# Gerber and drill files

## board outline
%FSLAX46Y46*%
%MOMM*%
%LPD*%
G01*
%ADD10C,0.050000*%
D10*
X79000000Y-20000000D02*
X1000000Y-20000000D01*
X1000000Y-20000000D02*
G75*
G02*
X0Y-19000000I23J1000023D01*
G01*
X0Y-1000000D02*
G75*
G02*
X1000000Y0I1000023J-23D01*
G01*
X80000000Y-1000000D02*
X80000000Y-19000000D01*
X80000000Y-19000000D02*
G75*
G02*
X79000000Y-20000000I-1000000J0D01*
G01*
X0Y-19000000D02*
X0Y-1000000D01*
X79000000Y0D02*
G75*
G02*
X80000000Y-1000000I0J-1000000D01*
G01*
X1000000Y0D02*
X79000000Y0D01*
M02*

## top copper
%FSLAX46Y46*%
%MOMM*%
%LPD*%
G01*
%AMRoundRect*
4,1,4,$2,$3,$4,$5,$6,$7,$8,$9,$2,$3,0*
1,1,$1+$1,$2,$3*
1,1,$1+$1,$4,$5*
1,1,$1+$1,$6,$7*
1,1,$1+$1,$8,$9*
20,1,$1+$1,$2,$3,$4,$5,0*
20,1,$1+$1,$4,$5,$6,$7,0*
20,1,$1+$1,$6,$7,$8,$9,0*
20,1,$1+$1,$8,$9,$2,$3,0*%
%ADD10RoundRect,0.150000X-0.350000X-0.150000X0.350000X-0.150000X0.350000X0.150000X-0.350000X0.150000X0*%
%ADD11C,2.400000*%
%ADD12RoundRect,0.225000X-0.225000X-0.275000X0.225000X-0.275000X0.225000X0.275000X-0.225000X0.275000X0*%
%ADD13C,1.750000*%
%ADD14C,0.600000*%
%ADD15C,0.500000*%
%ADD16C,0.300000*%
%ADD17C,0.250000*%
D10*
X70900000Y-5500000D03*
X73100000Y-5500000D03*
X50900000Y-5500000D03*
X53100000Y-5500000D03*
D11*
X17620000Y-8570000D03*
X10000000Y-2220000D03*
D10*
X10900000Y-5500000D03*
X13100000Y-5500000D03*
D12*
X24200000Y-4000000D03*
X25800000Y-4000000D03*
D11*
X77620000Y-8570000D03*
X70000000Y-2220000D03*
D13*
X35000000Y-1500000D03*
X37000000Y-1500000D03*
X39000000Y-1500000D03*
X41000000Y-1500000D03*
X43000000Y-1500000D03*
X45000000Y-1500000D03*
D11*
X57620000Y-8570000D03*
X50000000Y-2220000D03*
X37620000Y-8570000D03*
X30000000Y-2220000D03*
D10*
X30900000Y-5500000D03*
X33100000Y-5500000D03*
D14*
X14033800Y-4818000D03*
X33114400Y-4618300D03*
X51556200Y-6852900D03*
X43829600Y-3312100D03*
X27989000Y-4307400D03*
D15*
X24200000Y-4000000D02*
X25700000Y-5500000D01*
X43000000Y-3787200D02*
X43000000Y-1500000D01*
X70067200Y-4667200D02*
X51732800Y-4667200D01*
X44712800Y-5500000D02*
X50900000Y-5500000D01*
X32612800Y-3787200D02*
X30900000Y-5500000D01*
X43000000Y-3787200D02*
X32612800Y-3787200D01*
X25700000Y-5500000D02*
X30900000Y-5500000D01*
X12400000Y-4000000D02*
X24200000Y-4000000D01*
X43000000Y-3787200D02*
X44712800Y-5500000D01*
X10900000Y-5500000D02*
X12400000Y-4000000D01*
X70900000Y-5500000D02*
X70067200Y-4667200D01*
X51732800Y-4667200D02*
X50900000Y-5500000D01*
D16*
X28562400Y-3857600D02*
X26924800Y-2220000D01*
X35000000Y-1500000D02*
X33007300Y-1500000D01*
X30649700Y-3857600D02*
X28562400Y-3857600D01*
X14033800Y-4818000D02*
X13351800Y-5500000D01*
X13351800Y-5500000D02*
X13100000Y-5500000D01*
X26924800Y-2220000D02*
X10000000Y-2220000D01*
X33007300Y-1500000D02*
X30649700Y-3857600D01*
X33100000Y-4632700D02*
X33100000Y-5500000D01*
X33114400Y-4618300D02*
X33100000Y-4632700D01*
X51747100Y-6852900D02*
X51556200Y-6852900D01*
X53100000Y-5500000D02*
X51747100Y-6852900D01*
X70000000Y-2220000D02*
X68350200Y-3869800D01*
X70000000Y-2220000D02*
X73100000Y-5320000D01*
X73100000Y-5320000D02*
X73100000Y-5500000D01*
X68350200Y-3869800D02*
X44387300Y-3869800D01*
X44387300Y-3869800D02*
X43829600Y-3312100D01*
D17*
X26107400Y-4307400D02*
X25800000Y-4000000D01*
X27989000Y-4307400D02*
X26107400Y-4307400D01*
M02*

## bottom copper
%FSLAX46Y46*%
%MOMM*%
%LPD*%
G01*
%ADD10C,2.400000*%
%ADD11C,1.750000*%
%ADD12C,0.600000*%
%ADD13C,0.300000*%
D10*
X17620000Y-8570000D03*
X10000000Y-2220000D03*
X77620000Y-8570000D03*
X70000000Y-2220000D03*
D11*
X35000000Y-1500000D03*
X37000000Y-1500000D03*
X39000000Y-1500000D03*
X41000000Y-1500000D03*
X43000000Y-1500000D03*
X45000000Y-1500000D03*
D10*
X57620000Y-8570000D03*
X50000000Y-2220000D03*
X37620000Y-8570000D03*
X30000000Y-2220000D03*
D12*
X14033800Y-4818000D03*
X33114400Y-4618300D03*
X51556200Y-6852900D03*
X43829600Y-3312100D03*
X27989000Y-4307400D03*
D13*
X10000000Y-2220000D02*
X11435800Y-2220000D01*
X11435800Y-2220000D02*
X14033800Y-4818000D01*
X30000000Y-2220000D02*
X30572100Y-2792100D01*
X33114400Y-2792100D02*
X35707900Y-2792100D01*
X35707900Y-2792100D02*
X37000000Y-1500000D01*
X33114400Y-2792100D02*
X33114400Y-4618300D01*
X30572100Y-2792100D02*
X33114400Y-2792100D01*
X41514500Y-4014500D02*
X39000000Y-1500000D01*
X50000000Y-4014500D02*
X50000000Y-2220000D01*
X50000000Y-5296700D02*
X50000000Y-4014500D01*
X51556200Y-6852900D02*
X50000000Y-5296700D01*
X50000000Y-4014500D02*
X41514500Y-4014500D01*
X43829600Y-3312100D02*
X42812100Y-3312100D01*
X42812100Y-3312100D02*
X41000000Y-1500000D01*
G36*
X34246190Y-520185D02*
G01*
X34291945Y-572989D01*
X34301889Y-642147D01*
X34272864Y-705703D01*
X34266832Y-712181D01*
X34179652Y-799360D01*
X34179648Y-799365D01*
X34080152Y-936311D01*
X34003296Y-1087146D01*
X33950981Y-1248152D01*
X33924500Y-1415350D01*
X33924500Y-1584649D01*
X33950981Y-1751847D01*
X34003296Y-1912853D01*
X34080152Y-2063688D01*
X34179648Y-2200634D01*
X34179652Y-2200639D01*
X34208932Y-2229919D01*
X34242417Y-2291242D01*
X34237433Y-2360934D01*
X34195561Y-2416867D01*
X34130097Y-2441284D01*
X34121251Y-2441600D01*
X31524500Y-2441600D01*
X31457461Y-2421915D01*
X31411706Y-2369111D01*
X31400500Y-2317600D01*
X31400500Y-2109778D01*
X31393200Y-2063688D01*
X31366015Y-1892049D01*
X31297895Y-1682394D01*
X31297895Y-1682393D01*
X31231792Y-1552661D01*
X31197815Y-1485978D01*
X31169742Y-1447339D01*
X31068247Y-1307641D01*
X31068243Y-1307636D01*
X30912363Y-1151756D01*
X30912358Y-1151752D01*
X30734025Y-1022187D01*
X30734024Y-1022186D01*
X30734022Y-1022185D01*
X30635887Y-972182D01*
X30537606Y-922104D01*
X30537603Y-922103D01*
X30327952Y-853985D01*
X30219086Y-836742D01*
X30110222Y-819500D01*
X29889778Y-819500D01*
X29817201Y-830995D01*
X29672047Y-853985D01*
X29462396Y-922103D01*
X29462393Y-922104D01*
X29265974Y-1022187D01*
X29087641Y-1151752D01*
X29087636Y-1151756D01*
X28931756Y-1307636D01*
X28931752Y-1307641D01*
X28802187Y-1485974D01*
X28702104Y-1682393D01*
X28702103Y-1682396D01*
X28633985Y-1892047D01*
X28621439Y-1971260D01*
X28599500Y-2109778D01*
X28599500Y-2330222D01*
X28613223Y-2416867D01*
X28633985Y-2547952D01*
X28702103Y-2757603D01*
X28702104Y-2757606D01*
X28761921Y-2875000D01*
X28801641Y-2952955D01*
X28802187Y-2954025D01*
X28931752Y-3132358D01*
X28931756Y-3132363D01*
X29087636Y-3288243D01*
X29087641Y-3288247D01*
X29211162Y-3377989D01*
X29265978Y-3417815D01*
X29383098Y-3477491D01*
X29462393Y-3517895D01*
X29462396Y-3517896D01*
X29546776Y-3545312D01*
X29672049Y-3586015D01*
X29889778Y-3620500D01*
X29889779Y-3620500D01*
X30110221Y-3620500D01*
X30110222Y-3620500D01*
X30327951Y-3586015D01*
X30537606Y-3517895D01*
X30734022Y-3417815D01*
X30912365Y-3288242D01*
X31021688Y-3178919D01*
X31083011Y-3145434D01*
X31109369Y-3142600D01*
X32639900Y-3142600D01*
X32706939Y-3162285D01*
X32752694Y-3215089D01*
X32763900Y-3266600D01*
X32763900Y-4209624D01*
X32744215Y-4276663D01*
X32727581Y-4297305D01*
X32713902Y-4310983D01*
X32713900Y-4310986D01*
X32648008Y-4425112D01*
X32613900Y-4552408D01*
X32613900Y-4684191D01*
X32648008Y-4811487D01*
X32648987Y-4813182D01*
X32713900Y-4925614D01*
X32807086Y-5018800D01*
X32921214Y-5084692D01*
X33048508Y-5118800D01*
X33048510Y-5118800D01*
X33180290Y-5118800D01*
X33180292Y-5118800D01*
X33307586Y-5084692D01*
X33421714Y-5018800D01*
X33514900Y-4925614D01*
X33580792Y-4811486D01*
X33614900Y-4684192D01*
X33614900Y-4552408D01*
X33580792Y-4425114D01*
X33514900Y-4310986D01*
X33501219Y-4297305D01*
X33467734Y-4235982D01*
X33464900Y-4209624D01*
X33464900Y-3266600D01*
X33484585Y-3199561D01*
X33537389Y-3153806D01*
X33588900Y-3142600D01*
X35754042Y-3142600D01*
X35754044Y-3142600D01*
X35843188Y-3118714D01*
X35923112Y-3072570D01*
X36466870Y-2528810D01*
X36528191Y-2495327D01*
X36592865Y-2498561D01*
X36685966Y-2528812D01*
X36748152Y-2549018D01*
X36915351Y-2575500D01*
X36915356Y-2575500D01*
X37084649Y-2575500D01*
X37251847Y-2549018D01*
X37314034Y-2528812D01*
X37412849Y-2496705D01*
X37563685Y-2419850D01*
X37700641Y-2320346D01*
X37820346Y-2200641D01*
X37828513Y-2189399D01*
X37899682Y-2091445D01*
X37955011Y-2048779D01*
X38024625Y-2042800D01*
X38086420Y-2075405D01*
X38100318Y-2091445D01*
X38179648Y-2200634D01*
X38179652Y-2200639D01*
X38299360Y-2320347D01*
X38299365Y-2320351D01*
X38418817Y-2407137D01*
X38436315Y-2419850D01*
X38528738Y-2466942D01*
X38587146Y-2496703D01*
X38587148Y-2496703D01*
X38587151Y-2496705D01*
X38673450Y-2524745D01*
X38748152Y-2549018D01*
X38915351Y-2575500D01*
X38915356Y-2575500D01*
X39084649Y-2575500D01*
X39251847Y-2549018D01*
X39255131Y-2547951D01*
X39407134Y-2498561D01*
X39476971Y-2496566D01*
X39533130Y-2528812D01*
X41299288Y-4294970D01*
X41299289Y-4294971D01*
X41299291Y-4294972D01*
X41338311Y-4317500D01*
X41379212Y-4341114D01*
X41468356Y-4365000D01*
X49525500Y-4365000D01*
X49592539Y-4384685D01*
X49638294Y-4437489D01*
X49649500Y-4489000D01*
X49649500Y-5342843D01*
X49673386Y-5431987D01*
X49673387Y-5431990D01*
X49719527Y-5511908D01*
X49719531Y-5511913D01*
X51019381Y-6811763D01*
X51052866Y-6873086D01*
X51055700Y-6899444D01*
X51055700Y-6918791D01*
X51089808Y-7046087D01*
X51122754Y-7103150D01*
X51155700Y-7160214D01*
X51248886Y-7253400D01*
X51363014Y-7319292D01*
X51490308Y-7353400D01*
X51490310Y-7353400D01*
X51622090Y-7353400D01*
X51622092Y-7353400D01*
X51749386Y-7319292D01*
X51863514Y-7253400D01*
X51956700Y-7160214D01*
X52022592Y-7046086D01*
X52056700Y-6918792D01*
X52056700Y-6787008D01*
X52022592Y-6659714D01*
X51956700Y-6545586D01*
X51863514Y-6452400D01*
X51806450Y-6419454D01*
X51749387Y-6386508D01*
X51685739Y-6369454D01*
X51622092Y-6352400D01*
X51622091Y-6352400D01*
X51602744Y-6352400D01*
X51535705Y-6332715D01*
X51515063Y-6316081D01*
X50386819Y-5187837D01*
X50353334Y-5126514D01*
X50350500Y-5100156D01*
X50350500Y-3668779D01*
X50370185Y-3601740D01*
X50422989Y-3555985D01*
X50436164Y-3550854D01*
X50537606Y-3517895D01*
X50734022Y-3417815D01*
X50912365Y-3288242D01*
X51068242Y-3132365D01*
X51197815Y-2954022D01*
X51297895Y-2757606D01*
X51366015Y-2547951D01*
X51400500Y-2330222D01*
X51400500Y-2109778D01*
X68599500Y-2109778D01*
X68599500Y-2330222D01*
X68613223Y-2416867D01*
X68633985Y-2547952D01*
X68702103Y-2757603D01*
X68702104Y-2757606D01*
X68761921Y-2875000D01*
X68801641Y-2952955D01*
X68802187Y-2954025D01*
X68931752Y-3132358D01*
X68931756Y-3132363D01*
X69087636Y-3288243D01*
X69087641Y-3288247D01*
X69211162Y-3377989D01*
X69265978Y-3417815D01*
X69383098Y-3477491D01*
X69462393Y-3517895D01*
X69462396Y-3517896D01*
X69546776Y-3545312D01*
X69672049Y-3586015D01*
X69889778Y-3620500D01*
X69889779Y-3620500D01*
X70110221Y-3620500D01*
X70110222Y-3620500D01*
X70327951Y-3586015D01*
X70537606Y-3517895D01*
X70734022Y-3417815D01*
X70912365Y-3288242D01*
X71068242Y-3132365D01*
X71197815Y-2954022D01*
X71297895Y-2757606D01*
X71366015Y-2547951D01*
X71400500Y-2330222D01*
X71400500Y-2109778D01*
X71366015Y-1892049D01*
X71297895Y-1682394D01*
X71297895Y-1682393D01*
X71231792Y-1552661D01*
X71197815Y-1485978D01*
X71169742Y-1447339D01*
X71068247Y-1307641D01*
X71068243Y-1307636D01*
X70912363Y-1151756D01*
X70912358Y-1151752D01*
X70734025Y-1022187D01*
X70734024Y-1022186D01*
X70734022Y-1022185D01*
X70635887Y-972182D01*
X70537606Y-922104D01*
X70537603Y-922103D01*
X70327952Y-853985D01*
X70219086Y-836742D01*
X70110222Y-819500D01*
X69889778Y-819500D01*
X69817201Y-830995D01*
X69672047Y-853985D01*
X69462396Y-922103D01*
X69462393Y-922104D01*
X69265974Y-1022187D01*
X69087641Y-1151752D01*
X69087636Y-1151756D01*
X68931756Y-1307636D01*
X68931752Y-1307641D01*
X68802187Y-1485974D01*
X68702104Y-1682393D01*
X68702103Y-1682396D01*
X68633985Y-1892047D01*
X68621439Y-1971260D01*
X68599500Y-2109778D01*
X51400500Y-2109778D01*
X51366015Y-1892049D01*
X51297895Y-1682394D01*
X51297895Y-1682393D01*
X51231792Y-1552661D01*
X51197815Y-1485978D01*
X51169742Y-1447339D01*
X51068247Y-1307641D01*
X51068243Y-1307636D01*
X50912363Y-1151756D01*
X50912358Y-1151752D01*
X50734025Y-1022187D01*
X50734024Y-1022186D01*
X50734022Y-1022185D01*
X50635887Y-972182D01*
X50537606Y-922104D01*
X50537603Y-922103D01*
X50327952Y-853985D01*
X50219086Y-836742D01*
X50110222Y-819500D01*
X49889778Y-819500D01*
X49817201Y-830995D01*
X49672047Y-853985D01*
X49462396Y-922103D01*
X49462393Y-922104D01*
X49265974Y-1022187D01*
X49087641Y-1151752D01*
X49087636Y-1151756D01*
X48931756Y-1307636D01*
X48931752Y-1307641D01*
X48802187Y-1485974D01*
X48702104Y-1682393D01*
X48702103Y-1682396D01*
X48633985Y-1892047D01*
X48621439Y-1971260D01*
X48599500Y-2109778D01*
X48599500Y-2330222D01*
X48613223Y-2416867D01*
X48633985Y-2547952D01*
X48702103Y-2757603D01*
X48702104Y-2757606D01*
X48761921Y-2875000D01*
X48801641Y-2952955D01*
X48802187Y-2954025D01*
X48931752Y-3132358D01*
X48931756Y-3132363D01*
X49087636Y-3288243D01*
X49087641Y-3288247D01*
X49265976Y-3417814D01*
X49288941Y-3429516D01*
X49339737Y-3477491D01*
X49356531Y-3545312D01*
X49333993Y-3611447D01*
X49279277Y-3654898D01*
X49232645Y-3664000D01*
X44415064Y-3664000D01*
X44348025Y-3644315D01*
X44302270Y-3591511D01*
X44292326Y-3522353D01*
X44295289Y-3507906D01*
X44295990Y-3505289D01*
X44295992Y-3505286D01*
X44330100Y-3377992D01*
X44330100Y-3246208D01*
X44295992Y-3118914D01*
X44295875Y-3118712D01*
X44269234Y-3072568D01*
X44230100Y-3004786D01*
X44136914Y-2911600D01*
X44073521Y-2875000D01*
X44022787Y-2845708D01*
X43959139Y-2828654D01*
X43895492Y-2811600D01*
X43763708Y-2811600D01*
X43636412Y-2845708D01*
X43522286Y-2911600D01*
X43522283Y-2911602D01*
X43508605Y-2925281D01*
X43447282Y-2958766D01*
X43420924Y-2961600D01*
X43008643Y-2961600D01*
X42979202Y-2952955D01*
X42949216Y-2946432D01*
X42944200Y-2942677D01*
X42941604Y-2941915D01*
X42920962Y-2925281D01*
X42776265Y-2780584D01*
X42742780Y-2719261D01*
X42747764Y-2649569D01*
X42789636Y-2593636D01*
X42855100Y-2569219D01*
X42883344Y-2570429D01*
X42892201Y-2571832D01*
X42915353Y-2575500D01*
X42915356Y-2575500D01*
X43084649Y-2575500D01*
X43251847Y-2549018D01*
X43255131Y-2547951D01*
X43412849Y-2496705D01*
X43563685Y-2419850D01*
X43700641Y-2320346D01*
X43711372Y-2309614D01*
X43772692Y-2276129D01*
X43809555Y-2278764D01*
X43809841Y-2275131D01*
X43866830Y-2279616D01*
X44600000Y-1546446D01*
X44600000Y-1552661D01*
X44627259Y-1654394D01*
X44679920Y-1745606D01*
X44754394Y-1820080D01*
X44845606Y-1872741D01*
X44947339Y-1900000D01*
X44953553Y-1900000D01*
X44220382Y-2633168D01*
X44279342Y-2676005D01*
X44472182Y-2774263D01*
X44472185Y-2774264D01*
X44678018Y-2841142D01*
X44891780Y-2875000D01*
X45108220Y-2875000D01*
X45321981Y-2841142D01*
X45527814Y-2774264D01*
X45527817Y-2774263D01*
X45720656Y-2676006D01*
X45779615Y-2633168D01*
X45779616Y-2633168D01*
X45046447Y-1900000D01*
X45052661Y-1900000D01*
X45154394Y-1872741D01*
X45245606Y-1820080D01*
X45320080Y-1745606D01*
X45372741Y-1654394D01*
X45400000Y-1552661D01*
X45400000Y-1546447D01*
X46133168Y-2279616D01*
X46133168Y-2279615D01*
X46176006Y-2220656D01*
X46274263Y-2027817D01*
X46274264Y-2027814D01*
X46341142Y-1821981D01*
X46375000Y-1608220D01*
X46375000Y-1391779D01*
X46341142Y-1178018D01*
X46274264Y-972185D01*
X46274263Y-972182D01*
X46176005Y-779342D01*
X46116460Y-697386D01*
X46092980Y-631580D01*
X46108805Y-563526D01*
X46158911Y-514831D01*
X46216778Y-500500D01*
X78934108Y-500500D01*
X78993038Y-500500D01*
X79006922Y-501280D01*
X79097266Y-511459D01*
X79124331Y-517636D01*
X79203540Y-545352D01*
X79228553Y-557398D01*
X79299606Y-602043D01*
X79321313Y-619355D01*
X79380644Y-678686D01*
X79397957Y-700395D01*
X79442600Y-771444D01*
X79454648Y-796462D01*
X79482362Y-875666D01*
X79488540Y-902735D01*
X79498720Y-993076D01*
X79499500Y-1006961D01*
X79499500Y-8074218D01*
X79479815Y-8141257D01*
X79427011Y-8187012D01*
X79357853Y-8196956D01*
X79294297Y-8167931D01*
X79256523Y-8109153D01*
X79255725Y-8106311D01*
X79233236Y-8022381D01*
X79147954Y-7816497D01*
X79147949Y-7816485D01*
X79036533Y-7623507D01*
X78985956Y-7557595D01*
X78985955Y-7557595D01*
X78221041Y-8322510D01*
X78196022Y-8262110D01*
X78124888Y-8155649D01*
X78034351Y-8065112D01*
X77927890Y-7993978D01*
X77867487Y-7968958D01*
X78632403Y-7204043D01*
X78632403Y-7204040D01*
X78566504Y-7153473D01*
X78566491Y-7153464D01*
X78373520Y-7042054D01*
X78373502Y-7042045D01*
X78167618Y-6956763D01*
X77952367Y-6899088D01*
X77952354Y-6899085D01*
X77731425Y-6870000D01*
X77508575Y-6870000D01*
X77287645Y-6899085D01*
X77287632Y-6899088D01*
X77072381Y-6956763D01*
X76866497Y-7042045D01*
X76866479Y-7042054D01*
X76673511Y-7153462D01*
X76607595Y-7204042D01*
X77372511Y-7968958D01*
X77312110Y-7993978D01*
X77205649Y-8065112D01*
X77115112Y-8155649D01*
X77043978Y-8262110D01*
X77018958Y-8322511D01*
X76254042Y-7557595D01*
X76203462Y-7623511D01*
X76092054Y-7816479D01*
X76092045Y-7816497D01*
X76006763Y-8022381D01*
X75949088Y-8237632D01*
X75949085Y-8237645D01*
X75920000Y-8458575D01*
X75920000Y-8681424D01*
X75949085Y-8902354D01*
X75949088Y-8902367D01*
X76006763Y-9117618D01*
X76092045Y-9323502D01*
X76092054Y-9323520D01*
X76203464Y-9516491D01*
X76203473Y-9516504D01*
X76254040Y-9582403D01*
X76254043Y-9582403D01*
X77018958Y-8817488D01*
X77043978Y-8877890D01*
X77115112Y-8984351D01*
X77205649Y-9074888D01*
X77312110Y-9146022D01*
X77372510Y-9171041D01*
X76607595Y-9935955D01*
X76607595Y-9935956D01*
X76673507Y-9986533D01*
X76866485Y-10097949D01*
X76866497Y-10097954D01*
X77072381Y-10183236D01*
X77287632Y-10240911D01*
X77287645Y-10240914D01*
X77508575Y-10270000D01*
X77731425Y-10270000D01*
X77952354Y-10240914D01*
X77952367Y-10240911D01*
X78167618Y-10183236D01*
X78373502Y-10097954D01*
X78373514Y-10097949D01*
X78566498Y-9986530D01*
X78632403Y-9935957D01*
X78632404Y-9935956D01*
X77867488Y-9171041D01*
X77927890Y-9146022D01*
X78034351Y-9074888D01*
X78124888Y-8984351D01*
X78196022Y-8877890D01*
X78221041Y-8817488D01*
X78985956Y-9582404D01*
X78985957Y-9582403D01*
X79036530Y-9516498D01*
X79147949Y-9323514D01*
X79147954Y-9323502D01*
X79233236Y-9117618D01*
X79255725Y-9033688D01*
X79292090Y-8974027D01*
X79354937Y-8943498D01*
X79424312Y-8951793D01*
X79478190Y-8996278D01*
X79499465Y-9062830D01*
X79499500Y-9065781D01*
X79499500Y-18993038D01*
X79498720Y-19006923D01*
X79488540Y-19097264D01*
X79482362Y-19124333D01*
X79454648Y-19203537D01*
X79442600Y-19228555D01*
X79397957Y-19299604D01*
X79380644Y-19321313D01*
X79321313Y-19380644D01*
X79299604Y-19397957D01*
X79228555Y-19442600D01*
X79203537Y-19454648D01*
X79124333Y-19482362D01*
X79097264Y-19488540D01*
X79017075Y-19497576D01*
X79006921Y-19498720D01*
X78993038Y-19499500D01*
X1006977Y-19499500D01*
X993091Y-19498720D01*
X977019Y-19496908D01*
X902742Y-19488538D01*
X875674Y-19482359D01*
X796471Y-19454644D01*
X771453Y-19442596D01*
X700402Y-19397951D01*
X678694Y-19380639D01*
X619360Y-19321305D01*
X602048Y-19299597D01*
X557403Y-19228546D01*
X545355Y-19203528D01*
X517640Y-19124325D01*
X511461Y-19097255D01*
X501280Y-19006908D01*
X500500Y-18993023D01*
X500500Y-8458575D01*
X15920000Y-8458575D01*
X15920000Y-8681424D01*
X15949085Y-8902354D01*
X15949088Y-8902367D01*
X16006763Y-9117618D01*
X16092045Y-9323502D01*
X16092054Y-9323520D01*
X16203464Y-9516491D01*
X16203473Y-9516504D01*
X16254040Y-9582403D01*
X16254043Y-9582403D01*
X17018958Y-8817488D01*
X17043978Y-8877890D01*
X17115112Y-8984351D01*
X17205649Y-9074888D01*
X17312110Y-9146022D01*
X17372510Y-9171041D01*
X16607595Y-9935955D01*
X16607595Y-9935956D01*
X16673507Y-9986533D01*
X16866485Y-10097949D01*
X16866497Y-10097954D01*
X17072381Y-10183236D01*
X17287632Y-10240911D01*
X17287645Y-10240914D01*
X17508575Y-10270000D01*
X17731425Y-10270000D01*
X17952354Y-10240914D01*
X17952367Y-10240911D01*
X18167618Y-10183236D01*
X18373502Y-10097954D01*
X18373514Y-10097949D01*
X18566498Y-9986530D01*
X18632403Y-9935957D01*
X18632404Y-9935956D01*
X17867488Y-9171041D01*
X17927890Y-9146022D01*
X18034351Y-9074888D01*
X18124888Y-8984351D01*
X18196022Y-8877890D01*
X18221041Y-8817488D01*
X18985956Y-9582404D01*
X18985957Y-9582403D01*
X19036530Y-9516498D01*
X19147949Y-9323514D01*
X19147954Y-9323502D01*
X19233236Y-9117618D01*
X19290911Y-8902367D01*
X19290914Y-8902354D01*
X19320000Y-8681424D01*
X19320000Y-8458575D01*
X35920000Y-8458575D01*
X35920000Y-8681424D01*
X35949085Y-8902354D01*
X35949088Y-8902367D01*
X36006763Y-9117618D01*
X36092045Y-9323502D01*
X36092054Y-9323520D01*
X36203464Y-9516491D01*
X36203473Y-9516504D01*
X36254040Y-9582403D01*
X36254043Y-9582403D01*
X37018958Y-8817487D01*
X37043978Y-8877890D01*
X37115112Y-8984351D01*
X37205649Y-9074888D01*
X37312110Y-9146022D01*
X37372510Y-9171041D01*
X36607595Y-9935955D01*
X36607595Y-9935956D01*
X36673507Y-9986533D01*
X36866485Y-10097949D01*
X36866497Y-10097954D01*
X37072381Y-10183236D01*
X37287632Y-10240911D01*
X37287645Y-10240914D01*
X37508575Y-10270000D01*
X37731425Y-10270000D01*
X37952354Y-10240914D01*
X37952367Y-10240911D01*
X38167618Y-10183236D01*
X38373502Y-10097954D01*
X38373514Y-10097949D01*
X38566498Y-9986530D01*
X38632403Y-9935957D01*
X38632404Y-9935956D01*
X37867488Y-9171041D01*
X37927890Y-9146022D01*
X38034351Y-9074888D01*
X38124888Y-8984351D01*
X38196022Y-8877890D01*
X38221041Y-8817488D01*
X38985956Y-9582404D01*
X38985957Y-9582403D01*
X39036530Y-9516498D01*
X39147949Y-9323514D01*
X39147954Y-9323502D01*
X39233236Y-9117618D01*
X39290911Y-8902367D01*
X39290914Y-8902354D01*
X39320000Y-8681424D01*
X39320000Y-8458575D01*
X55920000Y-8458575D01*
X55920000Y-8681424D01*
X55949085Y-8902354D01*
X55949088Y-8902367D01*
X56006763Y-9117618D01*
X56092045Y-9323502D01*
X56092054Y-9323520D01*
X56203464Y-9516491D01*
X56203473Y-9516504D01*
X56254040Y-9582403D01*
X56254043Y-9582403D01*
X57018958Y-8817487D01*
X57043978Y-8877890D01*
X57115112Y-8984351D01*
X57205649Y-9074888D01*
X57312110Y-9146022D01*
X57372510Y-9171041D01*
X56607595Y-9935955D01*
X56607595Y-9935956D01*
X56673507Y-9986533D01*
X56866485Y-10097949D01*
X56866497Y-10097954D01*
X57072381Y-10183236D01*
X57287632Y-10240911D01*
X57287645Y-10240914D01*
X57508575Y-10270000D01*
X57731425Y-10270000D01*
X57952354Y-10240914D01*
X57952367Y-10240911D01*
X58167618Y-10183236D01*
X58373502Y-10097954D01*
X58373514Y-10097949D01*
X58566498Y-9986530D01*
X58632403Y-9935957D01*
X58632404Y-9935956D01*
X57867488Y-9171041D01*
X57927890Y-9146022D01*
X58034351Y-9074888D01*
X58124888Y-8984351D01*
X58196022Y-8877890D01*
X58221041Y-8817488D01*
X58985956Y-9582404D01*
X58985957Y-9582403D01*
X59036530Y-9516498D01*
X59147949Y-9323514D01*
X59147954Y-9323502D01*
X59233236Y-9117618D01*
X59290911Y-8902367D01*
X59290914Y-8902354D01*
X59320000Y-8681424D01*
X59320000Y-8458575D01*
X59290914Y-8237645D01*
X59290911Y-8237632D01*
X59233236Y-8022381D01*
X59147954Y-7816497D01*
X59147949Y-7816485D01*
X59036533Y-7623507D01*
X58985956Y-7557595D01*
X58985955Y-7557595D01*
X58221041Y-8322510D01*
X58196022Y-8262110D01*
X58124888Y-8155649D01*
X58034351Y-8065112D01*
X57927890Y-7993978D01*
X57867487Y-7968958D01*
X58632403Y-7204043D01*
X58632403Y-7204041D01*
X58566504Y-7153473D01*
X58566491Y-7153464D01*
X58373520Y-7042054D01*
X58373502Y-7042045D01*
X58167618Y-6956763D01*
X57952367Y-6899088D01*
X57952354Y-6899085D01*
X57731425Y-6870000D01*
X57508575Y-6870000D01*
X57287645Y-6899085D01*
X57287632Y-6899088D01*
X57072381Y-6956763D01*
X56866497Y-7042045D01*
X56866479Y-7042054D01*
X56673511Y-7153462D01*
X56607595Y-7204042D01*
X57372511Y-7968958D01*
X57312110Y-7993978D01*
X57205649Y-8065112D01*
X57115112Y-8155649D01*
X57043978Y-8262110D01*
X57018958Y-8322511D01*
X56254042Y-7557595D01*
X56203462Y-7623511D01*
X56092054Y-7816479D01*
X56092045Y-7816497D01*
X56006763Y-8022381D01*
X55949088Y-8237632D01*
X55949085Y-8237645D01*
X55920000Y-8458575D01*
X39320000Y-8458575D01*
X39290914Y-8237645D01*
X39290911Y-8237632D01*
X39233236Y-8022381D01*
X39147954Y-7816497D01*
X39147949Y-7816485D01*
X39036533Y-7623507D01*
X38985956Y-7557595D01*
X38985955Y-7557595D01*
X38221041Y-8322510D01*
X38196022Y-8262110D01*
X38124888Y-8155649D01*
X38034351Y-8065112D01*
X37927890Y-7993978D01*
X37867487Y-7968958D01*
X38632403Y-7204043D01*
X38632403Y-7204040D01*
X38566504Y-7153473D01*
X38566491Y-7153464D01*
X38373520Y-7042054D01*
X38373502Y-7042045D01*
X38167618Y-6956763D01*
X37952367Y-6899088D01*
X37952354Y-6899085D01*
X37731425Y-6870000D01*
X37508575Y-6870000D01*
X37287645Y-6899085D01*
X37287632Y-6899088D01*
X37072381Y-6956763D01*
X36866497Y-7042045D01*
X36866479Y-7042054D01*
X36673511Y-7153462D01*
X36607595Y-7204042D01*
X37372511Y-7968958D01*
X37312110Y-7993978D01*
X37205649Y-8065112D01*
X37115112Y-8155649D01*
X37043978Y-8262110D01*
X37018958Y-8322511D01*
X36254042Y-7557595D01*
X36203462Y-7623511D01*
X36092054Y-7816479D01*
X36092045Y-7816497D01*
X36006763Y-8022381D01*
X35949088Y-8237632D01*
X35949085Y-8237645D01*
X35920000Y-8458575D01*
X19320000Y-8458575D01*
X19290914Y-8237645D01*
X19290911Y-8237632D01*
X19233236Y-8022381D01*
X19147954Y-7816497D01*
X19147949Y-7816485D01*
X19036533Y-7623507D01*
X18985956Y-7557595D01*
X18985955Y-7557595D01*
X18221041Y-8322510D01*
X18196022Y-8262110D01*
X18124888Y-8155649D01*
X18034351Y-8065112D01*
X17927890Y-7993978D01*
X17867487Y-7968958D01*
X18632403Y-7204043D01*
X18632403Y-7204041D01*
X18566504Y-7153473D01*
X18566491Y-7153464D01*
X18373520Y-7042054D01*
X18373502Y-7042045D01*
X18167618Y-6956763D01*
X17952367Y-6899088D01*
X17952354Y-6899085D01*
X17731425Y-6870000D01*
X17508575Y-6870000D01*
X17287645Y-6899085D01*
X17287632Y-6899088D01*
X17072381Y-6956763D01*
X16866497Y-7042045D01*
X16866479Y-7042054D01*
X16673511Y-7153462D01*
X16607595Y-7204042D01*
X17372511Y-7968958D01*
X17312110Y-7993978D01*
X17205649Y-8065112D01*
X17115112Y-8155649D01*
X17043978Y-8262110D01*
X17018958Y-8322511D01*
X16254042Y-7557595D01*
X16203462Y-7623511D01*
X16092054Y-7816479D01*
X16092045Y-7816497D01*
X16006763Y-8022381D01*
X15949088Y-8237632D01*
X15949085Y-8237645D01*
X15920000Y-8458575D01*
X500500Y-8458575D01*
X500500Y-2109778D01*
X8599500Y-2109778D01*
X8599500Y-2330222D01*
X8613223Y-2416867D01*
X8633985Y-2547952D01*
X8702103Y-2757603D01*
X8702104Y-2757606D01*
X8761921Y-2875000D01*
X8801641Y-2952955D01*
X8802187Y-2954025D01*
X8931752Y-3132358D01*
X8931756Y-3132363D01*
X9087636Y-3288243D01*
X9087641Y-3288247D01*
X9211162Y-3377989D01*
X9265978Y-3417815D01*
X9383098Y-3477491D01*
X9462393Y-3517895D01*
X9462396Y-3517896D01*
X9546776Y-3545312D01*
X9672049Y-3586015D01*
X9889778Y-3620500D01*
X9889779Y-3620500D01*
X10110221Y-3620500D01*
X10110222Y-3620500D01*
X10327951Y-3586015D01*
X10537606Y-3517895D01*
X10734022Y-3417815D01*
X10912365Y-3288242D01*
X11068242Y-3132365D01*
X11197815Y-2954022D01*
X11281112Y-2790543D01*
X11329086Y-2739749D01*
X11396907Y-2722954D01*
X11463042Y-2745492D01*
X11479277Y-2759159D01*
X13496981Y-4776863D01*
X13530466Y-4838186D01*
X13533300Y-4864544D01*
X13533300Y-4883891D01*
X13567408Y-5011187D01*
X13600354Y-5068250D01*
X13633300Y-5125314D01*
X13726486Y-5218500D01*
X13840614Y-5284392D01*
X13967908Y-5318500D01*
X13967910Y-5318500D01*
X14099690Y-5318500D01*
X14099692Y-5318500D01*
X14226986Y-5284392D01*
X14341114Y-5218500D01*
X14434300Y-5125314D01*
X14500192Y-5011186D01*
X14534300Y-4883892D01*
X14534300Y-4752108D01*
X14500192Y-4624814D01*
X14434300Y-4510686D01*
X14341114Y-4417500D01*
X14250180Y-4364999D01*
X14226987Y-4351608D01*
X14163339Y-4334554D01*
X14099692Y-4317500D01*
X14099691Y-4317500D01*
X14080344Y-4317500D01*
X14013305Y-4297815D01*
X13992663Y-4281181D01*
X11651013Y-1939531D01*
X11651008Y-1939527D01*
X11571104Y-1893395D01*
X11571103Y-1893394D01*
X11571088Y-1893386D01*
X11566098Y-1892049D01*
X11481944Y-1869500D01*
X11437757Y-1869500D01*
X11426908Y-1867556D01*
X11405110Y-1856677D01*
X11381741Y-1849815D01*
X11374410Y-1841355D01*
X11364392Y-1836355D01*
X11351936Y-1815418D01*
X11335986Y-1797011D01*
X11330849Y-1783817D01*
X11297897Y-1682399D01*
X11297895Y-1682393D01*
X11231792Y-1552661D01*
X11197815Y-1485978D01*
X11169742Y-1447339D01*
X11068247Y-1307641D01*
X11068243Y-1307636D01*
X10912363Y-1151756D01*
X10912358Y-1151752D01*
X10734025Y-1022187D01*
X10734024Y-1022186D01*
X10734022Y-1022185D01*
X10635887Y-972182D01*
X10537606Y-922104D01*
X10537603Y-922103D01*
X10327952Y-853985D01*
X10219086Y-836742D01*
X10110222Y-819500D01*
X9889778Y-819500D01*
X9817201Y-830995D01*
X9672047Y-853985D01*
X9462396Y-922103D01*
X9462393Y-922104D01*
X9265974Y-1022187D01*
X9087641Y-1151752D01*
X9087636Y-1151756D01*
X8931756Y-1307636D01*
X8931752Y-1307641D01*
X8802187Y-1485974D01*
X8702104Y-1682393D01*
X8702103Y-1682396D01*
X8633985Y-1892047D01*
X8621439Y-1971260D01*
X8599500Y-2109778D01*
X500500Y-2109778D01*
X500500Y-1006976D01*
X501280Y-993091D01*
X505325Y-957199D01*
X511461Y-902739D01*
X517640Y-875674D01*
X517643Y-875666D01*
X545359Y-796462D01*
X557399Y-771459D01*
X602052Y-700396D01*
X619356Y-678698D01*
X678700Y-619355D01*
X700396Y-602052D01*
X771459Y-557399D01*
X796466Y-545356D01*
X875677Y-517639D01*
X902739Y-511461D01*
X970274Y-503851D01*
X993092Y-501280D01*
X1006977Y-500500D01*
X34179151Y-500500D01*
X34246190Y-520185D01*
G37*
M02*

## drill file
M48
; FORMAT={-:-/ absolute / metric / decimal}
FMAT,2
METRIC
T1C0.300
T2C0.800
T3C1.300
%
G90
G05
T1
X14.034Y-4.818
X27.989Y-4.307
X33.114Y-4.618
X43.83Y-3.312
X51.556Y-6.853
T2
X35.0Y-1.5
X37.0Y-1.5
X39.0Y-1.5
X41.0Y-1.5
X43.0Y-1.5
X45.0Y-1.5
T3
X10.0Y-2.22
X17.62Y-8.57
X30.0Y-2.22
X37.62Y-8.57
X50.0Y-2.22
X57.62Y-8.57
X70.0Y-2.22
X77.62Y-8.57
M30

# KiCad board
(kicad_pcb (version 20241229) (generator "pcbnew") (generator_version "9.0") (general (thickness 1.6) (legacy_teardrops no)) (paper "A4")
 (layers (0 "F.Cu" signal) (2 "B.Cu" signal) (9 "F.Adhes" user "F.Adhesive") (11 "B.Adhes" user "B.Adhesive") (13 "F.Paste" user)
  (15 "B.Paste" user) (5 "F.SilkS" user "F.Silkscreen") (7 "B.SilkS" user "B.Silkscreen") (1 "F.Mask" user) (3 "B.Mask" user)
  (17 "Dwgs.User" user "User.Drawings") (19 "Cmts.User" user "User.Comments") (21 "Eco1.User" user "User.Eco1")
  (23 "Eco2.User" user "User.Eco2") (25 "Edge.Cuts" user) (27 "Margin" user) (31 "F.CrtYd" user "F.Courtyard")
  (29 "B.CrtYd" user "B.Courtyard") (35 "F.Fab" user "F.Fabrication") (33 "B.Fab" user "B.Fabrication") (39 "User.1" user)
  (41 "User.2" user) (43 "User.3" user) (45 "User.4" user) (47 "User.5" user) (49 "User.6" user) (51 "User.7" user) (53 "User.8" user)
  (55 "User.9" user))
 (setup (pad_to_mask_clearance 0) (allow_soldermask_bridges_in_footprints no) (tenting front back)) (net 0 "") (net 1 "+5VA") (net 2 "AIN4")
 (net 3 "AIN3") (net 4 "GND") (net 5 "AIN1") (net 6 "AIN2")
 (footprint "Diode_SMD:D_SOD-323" (layer "F.Cu") (at 72 5.5)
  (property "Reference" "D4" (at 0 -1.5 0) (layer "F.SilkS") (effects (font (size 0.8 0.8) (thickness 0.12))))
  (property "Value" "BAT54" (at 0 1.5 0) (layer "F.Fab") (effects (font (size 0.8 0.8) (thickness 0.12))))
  (pad "1" smd roundrect (at -1.1 0) (size 1 0.6) (layers "F.Cu" "F.Mask") (roundrect_rratio 0.25) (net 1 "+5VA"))
  (pad "2" smd roundrect (at 1.1 0) (size 1 0.6) (layers "F.Cu" "F.Mask") (roundrect_rratio 0.25) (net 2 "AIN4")))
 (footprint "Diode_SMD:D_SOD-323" (layer "F.Cu") (at 52 5.5)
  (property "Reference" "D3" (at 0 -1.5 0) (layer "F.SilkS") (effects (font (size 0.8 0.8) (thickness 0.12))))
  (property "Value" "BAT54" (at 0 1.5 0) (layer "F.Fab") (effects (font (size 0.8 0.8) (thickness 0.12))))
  (pad "1" smd roundrect (at -1.1 0) (size 1 0.6) (layers "F.Cu" "F.Mask") (roundrect_rratio 0.25) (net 1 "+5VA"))
  (pad "2" smd roundrect (at 1.1 0) (size 1 0.6) (layers "F.Cu" "F.Mask") (roundrect_rratio 0.25) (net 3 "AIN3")))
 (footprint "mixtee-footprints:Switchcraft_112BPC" (layer "F.Cu") (at 10 20 90)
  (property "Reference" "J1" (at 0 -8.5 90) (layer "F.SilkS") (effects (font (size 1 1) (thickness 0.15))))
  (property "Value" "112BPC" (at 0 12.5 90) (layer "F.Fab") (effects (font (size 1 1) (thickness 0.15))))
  (pad "S" thru_hole circle (at 11.43 7.62) (size 2.4 2.4) (drill 1.3) (layers "*.Cu" "*.Mask") (remove_unused_layers no) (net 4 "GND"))
  (pad "T" thru_hole circle (at 17.78 0) (size 2.4 2.4) (drill 1.3) (layers "*.Cu" "*.Mask") (remove_unused_layers no) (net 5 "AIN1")))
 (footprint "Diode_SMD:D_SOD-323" (layer "F.Cu") (at 12 5.5)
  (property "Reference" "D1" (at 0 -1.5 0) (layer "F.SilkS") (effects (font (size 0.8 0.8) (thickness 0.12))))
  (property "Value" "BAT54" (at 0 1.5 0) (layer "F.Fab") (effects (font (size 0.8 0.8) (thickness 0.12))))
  (pad "1" smd roundrect (at -1.1 0) (size 1 0.6) (layers "F.Cu" "F.Mask") (roundrect_rratio 0.25) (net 1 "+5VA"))
  (pad "2" smd roundrect (at 1.1 0) (size 1 0.6) (layers "F.Cu" "F.Mask") (roundrect_rratio 0.25) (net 5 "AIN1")))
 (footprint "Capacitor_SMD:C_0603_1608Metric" (layer "F.Cu") (at 25 4)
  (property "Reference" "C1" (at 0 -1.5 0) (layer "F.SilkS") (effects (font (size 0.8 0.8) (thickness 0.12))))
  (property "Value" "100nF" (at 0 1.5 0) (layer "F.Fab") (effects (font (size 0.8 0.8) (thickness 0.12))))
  (pad "1" smd roundrect (at -0.8 0) (size 0.9 1) (layers "F.Cu" "F.Mask") (roundrect_rratio 0.25) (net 1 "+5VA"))
  (pad "2" smd roundrect (at 0.8 0) (size 0.9 1) (layers "F.Cu" "F.Mask") (roundrect_rratio 0.25) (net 4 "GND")))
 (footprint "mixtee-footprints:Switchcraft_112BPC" (layer "F.Cu") (at 70 20 90)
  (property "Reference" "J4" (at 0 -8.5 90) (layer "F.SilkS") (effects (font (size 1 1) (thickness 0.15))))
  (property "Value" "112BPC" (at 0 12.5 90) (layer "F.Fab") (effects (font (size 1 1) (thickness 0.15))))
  (pad "S" thru_hole circle (at 11.43 7.62) (size 2.4 2.4) (drill 1.3) (layers "*.Cu" "*.Mask") (remove_unused_layers no) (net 4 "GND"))
  (pad "T" thru_hole circle (at 17.78 0) (size 2.4 2.4) (drill 1.3) (layers "*.Cu" "*.Mask") (remove_unused_layers no) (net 2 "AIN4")))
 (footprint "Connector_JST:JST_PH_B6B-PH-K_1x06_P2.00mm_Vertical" (layer "F.Cu") (at 35 1.5)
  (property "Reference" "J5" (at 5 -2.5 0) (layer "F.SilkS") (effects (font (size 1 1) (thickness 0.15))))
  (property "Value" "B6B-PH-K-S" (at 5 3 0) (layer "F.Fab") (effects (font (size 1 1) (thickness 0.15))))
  (pad "1" thru_hole circle (at 0 0) (size 1.75 1.75) (drill 0.8) (layers "*.Cu" "*.Mask") (remove_unused_layers no) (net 5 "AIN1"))
  (pad "2" thru_hole circle (at 2 0) (size 1.75 1.75) (drill 0.8) (layers "*.Cu" "*.Mask") (remove_unused_layers no) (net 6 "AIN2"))
  (pad "3" thru_hole circle (at 4 0) (size 1.75 1.75) (drill 0.8) (layers "*.Cu" "*.Mask") (remove_unused_layers no) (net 3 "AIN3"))
  (pad "4" thru_hole circle (at 6 0) (size 1.75 1.75) (drill 0.8) (layers "*.Cu" "*.Mask") (remove_unused_layers no) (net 2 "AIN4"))
  (pad "5" thru_hole circle (at 8 0) (size 1.75 1.75) (drill 0.8) (layers "*.Cu" "*.Mask") (remove_unused_layers no) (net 1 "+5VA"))
  (pad "6" thru_hole circle (at 10 0) (size 1.75 1.75) (drill 0.8) (layers "*.Cu" "*.Mask") (remove_unused_layers no) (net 4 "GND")))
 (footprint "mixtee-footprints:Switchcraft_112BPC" (layer "F.Cu") (at 50 20 90)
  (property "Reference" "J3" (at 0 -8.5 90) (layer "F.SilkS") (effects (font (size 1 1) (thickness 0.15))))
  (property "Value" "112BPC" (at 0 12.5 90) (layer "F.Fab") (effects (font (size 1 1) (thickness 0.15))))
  (pad "S" thru_hole circle (at 11.43 7.62) (size 2.4 2.4) (drill 1.3) (layers "*.Cu" "*.Mask") (remove_unused_layers no) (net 4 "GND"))
  (pad "T" thru_hole circle (at 17.78 0) (size 2.4 2.4) (drill 1.3) (layers "*.Cu" "*.Mask") (remove_unused_layers no) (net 3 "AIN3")))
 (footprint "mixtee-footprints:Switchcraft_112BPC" (layer "F.Cu") (at 30 20 90)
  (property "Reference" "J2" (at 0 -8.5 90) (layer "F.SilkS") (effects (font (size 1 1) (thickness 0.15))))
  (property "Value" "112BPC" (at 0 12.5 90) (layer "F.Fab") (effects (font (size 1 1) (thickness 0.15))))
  (pad "S" thru_hole circle (at 11.43 7.62) (size 2.4 2.4) (drill 1.3) (layers "*.Cu" "*.Mask") (remove_unused_layers no) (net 4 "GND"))
  (pad "T" thru_hole circle (at 17.78 0) (size 2.4 2.4) (drill 1.3) (layers "*.Cu" "*.Mask") (remove_unused_layers no) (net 6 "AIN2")))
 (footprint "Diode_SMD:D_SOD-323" (layer "F.Cu") (at 32 5.5)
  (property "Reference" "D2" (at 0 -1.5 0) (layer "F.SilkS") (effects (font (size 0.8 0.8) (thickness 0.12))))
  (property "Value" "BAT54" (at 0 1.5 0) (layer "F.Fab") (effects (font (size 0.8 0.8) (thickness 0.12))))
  (pad "1" smd roundrect (at -1.1 0) (size 1 0.6) (layers "F.Cu" "F.Mask") (roundrect_rratio 0.25) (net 1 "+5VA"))
  (pad "2" smd roundrect (at 1.1 0) (size 1 0.6) (layers "F.Cu" "F.Mask") (roundrect_rratio 0.25) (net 6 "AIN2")))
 (gr_line (start 79 20) (end 1 20) (stroke (width 0.05) (type solid)) (layer "Edge.Cuts"))
 (gr_arc (start 1 20) (mid 0.2929 19.7071) (end 0 19) (stroke (width 0.05) (type solid)) (layer "Edge.Cuts"))
 (gr_arc (start 0 1) (mid 0.2929 0.2929) (end 1 0) (stroke (width 0.05) (type solid)) (layer "Edge.Cuts"))
 (gr_line (start 80 1) (end 80 19) (stroke (width 0.05) (type solid)) (layer "Edge.Cuts"))
 (gr_arc (start 80 19) (mid 79.7071 19.7071) (end 79 20) (stroke (width 0.05) (type solid)) (layer "Edge.Cuts"))
 (gr_line (start 0 19) (end 0 1) (stroke (width 0.05) (type solid)) (layer "Edge.Cuts"))
 (gr_arc (start 79 0) (mid 79.7071 0.2929) (end 80 1) (stroke (width 0.05) (type solid)) (layer "Edge.Cuts"))
 (gr_line (start 1 0) (end 79 0) (stroke (width 0.05) (type solid)) (layer "Edge.Cuts"))
 (segment (start 24.2 4) (end 25.7 5.5) (width 0.5) (layer "F.Cu") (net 1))
 (segment (start 43 3.7872) (end 43 1.5) (width 0.5) (layer "F.Cu") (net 1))
 (segment (start 70.0672 4.6672) (end 51.7328 4.6672) (width 0.5) (layer "F.Cu") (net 1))
 (segment (start 44.7128 5.5) (end 50.9 5.5) (width 0.5) (layer "F.Cu") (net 1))
 (segment (start 32.6128 3.7872) (end 30.9 5.5) (width 0.5) (layer "F.Cu") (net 1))
 (segment (start 43 3.7872) (end 32.6128 3.7872) (width 0.5) (layer "F.Cu") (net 1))
 (segment (start 25.7 5.5) (end 30.9 5.5) (width 0.5) (layer "F.Cu") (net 1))
 (segment (start 12.4 4) (end 24.2 4) (width 0.5) (layer "F.Cu") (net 1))
 (segment (start 43 3.7872) (end 44.7128 5.5) (width 0.5) (layer "F.Cu") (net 1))
 (segment (start 10.9 5.5) (end 12.4 4) (width 0.5) (layer "F.Cu") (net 1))
 (segment (start 70.9 5.5) (end 70.0672 4.6672) (width 0.5) (layer "F.Cu") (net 1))
 (segment (start 51.7328 4.6672) (end 50.9 5.5) (width 0.5) (layer "F.Cu") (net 1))
 (segment (start 28.5624 3.8576) (end 26.9248 2.22) (width 0.3) (layer "F.Cu") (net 5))
 (segment (start 35 1.5) (end 33.0073 1.5) (width 0.3) (layer "F.Cu") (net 5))
 (segment (start 30.6497 3.8576) (end 28.5624 3.8576) (width 0.3) (layer "F.Cu") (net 5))
 (segment (start 14.0338 4.818) (end 13.3518 5.5) (width 0.3) (layer "F.Cu") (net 5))
 (segment (start 13.3518 5.5) (end 13.1 5.5) (width 0.3) (layer "F.Cu") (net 5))
 (segment (start 26.9248 2.22) (end 10 2.22) (width 0.3) (layer "F.Cu") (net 5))
 (segment (start 33.0073 1.5) (end 30.6497 3.8576) (width 0.3) (layer "F.Cu") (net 5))
 (via (at 14.0338 4.818) (size 0.6) (drill 0.3) (layers "F.Cu" "B.Cu") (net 5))
 (segment (start 10 2.22) (end 11.4358 2.22) (width 0.3) (layer "B.Cu") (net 5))
 (segment (start 11.4358 2.22) (end 14.0338 4.818) (width 0.3) (layer "B.Cu") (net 5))
 (segment (start 33.1 4.6327) (end 33.1 5.5) (width 0.3) (layer "F.Cu") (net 6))
 (segment (start 33.1144 4.6183) (end 33.1 4.6327) (width 0.3) (layer "F.Cu") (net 6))
 (via (at 33.1144 4.6183) (size 0.6) (drill 0.3) (layers "F.Cu" "B.Cu") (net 6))
 (segment (start 30 2.22) (end 30.5721 2.7921) (width 0.3) (layer "B.Cu") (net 6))
 (segment (start 33.1144 2.7921) (end 35.7079 2.7921) (width 0.3) (layer "B.Cu") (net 6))
 (segment (start 35.7079 2.7921) (end 37 1.5) (width 0.3) (layer "B.Cu") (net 6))
 (segment (start 33.1144 2.7921) (end 33.1144 4.6183) (width 0.3) (layer "B.Cu") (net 6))
 (segment (start 30.5721 2.7921) (end 33.1144 2.7921) (width 0.3) (layer "B.Cu") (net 6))
 (segment (start 51.7471 6.8529) (end 51.5562 6.8529) (width 0.3) (layer "F.Cu") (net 3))
 (segment (start 53.1 5.5) (end 51.7471 6.8529) (width 0.3) (layer "F.Cu") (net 3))
 (via (at 51.5562 6.8529) (size 0.6) (drill 0.3) (layers "F.Cu" "B.Cu") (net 3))
 (segment (start 41.5145 4.0145) (end 39 1.5) (width 0.3) (layer "B.Cu") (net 3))
 (segment (start 50 4.0145) (end 50 2.22) (width 0.3) (layer "B.Cu") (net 3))
 (segment (start 50 5.2967) (end 50 4.0145) (width 0.3) (layer "B.Cu") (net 3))
 (segment (start 51.5562 6.8529) (end 50 5.2967) (width 0.3) (layer "B.Cu") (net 3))
 (segment (start 50 4.0145) (end 41.5145 4.0145) (width 0.3) (layer "B.Cu") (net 3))
 (segment (start 70 2.22) (end 68.3502 3.8698) (width 0.3) (layer "F.Cu") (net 2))
 (segment (start 70 2.22) (end 73.1 5.32) (width 0.3) (layer "F.Cu") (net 2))
 (segment (start 73.1 5.32) (end 73.1 5.5) (width 0.3) (layer "F.Cu") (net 2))
 (segment (start 68.3502 3.8698) (end 44.3873 3.8698) (width 0.3) (layer "F.Cu") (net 2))
 (segment (start 44.3873 3.8698) (end 43.8296 3.3121) (width 0.3) (layer "F.Cu") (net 2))
 (via (at 43.8296 3.3121) (size 0.6) (drill 0.3) (layers "F.Cu" "B.Cu") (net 2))
 (segment (start 43.8296 3.3121) (end 42.8121 3.3121) (width 0.3) (layer "B.Cu") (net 2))
 (segment (start 42.8121 3.3121) (end 41 1.5) (width 0.3) (layer "B.Cu") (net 2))
 (segment (start 26.1074 4.3074) (end 25.8 4) (width 0.25) (layer "F.Cu") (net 4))
 (segment (start 27.989 4.3074) (end 26.1074 4.3074) (width 0.25) (layer "F.Cu") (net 4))
 (via (at 27.989 4.3074) (size 0.6) (drill 0.3) (layers "F.Cu" "B.Cu") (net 4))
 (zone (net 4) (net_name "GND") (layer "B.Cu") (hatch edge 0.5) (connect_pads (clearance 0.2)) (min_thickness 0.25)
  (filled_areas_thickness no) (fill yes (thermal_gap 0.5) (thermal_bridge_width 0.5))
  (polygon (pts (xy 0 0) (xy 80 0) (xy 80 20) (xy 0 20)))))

